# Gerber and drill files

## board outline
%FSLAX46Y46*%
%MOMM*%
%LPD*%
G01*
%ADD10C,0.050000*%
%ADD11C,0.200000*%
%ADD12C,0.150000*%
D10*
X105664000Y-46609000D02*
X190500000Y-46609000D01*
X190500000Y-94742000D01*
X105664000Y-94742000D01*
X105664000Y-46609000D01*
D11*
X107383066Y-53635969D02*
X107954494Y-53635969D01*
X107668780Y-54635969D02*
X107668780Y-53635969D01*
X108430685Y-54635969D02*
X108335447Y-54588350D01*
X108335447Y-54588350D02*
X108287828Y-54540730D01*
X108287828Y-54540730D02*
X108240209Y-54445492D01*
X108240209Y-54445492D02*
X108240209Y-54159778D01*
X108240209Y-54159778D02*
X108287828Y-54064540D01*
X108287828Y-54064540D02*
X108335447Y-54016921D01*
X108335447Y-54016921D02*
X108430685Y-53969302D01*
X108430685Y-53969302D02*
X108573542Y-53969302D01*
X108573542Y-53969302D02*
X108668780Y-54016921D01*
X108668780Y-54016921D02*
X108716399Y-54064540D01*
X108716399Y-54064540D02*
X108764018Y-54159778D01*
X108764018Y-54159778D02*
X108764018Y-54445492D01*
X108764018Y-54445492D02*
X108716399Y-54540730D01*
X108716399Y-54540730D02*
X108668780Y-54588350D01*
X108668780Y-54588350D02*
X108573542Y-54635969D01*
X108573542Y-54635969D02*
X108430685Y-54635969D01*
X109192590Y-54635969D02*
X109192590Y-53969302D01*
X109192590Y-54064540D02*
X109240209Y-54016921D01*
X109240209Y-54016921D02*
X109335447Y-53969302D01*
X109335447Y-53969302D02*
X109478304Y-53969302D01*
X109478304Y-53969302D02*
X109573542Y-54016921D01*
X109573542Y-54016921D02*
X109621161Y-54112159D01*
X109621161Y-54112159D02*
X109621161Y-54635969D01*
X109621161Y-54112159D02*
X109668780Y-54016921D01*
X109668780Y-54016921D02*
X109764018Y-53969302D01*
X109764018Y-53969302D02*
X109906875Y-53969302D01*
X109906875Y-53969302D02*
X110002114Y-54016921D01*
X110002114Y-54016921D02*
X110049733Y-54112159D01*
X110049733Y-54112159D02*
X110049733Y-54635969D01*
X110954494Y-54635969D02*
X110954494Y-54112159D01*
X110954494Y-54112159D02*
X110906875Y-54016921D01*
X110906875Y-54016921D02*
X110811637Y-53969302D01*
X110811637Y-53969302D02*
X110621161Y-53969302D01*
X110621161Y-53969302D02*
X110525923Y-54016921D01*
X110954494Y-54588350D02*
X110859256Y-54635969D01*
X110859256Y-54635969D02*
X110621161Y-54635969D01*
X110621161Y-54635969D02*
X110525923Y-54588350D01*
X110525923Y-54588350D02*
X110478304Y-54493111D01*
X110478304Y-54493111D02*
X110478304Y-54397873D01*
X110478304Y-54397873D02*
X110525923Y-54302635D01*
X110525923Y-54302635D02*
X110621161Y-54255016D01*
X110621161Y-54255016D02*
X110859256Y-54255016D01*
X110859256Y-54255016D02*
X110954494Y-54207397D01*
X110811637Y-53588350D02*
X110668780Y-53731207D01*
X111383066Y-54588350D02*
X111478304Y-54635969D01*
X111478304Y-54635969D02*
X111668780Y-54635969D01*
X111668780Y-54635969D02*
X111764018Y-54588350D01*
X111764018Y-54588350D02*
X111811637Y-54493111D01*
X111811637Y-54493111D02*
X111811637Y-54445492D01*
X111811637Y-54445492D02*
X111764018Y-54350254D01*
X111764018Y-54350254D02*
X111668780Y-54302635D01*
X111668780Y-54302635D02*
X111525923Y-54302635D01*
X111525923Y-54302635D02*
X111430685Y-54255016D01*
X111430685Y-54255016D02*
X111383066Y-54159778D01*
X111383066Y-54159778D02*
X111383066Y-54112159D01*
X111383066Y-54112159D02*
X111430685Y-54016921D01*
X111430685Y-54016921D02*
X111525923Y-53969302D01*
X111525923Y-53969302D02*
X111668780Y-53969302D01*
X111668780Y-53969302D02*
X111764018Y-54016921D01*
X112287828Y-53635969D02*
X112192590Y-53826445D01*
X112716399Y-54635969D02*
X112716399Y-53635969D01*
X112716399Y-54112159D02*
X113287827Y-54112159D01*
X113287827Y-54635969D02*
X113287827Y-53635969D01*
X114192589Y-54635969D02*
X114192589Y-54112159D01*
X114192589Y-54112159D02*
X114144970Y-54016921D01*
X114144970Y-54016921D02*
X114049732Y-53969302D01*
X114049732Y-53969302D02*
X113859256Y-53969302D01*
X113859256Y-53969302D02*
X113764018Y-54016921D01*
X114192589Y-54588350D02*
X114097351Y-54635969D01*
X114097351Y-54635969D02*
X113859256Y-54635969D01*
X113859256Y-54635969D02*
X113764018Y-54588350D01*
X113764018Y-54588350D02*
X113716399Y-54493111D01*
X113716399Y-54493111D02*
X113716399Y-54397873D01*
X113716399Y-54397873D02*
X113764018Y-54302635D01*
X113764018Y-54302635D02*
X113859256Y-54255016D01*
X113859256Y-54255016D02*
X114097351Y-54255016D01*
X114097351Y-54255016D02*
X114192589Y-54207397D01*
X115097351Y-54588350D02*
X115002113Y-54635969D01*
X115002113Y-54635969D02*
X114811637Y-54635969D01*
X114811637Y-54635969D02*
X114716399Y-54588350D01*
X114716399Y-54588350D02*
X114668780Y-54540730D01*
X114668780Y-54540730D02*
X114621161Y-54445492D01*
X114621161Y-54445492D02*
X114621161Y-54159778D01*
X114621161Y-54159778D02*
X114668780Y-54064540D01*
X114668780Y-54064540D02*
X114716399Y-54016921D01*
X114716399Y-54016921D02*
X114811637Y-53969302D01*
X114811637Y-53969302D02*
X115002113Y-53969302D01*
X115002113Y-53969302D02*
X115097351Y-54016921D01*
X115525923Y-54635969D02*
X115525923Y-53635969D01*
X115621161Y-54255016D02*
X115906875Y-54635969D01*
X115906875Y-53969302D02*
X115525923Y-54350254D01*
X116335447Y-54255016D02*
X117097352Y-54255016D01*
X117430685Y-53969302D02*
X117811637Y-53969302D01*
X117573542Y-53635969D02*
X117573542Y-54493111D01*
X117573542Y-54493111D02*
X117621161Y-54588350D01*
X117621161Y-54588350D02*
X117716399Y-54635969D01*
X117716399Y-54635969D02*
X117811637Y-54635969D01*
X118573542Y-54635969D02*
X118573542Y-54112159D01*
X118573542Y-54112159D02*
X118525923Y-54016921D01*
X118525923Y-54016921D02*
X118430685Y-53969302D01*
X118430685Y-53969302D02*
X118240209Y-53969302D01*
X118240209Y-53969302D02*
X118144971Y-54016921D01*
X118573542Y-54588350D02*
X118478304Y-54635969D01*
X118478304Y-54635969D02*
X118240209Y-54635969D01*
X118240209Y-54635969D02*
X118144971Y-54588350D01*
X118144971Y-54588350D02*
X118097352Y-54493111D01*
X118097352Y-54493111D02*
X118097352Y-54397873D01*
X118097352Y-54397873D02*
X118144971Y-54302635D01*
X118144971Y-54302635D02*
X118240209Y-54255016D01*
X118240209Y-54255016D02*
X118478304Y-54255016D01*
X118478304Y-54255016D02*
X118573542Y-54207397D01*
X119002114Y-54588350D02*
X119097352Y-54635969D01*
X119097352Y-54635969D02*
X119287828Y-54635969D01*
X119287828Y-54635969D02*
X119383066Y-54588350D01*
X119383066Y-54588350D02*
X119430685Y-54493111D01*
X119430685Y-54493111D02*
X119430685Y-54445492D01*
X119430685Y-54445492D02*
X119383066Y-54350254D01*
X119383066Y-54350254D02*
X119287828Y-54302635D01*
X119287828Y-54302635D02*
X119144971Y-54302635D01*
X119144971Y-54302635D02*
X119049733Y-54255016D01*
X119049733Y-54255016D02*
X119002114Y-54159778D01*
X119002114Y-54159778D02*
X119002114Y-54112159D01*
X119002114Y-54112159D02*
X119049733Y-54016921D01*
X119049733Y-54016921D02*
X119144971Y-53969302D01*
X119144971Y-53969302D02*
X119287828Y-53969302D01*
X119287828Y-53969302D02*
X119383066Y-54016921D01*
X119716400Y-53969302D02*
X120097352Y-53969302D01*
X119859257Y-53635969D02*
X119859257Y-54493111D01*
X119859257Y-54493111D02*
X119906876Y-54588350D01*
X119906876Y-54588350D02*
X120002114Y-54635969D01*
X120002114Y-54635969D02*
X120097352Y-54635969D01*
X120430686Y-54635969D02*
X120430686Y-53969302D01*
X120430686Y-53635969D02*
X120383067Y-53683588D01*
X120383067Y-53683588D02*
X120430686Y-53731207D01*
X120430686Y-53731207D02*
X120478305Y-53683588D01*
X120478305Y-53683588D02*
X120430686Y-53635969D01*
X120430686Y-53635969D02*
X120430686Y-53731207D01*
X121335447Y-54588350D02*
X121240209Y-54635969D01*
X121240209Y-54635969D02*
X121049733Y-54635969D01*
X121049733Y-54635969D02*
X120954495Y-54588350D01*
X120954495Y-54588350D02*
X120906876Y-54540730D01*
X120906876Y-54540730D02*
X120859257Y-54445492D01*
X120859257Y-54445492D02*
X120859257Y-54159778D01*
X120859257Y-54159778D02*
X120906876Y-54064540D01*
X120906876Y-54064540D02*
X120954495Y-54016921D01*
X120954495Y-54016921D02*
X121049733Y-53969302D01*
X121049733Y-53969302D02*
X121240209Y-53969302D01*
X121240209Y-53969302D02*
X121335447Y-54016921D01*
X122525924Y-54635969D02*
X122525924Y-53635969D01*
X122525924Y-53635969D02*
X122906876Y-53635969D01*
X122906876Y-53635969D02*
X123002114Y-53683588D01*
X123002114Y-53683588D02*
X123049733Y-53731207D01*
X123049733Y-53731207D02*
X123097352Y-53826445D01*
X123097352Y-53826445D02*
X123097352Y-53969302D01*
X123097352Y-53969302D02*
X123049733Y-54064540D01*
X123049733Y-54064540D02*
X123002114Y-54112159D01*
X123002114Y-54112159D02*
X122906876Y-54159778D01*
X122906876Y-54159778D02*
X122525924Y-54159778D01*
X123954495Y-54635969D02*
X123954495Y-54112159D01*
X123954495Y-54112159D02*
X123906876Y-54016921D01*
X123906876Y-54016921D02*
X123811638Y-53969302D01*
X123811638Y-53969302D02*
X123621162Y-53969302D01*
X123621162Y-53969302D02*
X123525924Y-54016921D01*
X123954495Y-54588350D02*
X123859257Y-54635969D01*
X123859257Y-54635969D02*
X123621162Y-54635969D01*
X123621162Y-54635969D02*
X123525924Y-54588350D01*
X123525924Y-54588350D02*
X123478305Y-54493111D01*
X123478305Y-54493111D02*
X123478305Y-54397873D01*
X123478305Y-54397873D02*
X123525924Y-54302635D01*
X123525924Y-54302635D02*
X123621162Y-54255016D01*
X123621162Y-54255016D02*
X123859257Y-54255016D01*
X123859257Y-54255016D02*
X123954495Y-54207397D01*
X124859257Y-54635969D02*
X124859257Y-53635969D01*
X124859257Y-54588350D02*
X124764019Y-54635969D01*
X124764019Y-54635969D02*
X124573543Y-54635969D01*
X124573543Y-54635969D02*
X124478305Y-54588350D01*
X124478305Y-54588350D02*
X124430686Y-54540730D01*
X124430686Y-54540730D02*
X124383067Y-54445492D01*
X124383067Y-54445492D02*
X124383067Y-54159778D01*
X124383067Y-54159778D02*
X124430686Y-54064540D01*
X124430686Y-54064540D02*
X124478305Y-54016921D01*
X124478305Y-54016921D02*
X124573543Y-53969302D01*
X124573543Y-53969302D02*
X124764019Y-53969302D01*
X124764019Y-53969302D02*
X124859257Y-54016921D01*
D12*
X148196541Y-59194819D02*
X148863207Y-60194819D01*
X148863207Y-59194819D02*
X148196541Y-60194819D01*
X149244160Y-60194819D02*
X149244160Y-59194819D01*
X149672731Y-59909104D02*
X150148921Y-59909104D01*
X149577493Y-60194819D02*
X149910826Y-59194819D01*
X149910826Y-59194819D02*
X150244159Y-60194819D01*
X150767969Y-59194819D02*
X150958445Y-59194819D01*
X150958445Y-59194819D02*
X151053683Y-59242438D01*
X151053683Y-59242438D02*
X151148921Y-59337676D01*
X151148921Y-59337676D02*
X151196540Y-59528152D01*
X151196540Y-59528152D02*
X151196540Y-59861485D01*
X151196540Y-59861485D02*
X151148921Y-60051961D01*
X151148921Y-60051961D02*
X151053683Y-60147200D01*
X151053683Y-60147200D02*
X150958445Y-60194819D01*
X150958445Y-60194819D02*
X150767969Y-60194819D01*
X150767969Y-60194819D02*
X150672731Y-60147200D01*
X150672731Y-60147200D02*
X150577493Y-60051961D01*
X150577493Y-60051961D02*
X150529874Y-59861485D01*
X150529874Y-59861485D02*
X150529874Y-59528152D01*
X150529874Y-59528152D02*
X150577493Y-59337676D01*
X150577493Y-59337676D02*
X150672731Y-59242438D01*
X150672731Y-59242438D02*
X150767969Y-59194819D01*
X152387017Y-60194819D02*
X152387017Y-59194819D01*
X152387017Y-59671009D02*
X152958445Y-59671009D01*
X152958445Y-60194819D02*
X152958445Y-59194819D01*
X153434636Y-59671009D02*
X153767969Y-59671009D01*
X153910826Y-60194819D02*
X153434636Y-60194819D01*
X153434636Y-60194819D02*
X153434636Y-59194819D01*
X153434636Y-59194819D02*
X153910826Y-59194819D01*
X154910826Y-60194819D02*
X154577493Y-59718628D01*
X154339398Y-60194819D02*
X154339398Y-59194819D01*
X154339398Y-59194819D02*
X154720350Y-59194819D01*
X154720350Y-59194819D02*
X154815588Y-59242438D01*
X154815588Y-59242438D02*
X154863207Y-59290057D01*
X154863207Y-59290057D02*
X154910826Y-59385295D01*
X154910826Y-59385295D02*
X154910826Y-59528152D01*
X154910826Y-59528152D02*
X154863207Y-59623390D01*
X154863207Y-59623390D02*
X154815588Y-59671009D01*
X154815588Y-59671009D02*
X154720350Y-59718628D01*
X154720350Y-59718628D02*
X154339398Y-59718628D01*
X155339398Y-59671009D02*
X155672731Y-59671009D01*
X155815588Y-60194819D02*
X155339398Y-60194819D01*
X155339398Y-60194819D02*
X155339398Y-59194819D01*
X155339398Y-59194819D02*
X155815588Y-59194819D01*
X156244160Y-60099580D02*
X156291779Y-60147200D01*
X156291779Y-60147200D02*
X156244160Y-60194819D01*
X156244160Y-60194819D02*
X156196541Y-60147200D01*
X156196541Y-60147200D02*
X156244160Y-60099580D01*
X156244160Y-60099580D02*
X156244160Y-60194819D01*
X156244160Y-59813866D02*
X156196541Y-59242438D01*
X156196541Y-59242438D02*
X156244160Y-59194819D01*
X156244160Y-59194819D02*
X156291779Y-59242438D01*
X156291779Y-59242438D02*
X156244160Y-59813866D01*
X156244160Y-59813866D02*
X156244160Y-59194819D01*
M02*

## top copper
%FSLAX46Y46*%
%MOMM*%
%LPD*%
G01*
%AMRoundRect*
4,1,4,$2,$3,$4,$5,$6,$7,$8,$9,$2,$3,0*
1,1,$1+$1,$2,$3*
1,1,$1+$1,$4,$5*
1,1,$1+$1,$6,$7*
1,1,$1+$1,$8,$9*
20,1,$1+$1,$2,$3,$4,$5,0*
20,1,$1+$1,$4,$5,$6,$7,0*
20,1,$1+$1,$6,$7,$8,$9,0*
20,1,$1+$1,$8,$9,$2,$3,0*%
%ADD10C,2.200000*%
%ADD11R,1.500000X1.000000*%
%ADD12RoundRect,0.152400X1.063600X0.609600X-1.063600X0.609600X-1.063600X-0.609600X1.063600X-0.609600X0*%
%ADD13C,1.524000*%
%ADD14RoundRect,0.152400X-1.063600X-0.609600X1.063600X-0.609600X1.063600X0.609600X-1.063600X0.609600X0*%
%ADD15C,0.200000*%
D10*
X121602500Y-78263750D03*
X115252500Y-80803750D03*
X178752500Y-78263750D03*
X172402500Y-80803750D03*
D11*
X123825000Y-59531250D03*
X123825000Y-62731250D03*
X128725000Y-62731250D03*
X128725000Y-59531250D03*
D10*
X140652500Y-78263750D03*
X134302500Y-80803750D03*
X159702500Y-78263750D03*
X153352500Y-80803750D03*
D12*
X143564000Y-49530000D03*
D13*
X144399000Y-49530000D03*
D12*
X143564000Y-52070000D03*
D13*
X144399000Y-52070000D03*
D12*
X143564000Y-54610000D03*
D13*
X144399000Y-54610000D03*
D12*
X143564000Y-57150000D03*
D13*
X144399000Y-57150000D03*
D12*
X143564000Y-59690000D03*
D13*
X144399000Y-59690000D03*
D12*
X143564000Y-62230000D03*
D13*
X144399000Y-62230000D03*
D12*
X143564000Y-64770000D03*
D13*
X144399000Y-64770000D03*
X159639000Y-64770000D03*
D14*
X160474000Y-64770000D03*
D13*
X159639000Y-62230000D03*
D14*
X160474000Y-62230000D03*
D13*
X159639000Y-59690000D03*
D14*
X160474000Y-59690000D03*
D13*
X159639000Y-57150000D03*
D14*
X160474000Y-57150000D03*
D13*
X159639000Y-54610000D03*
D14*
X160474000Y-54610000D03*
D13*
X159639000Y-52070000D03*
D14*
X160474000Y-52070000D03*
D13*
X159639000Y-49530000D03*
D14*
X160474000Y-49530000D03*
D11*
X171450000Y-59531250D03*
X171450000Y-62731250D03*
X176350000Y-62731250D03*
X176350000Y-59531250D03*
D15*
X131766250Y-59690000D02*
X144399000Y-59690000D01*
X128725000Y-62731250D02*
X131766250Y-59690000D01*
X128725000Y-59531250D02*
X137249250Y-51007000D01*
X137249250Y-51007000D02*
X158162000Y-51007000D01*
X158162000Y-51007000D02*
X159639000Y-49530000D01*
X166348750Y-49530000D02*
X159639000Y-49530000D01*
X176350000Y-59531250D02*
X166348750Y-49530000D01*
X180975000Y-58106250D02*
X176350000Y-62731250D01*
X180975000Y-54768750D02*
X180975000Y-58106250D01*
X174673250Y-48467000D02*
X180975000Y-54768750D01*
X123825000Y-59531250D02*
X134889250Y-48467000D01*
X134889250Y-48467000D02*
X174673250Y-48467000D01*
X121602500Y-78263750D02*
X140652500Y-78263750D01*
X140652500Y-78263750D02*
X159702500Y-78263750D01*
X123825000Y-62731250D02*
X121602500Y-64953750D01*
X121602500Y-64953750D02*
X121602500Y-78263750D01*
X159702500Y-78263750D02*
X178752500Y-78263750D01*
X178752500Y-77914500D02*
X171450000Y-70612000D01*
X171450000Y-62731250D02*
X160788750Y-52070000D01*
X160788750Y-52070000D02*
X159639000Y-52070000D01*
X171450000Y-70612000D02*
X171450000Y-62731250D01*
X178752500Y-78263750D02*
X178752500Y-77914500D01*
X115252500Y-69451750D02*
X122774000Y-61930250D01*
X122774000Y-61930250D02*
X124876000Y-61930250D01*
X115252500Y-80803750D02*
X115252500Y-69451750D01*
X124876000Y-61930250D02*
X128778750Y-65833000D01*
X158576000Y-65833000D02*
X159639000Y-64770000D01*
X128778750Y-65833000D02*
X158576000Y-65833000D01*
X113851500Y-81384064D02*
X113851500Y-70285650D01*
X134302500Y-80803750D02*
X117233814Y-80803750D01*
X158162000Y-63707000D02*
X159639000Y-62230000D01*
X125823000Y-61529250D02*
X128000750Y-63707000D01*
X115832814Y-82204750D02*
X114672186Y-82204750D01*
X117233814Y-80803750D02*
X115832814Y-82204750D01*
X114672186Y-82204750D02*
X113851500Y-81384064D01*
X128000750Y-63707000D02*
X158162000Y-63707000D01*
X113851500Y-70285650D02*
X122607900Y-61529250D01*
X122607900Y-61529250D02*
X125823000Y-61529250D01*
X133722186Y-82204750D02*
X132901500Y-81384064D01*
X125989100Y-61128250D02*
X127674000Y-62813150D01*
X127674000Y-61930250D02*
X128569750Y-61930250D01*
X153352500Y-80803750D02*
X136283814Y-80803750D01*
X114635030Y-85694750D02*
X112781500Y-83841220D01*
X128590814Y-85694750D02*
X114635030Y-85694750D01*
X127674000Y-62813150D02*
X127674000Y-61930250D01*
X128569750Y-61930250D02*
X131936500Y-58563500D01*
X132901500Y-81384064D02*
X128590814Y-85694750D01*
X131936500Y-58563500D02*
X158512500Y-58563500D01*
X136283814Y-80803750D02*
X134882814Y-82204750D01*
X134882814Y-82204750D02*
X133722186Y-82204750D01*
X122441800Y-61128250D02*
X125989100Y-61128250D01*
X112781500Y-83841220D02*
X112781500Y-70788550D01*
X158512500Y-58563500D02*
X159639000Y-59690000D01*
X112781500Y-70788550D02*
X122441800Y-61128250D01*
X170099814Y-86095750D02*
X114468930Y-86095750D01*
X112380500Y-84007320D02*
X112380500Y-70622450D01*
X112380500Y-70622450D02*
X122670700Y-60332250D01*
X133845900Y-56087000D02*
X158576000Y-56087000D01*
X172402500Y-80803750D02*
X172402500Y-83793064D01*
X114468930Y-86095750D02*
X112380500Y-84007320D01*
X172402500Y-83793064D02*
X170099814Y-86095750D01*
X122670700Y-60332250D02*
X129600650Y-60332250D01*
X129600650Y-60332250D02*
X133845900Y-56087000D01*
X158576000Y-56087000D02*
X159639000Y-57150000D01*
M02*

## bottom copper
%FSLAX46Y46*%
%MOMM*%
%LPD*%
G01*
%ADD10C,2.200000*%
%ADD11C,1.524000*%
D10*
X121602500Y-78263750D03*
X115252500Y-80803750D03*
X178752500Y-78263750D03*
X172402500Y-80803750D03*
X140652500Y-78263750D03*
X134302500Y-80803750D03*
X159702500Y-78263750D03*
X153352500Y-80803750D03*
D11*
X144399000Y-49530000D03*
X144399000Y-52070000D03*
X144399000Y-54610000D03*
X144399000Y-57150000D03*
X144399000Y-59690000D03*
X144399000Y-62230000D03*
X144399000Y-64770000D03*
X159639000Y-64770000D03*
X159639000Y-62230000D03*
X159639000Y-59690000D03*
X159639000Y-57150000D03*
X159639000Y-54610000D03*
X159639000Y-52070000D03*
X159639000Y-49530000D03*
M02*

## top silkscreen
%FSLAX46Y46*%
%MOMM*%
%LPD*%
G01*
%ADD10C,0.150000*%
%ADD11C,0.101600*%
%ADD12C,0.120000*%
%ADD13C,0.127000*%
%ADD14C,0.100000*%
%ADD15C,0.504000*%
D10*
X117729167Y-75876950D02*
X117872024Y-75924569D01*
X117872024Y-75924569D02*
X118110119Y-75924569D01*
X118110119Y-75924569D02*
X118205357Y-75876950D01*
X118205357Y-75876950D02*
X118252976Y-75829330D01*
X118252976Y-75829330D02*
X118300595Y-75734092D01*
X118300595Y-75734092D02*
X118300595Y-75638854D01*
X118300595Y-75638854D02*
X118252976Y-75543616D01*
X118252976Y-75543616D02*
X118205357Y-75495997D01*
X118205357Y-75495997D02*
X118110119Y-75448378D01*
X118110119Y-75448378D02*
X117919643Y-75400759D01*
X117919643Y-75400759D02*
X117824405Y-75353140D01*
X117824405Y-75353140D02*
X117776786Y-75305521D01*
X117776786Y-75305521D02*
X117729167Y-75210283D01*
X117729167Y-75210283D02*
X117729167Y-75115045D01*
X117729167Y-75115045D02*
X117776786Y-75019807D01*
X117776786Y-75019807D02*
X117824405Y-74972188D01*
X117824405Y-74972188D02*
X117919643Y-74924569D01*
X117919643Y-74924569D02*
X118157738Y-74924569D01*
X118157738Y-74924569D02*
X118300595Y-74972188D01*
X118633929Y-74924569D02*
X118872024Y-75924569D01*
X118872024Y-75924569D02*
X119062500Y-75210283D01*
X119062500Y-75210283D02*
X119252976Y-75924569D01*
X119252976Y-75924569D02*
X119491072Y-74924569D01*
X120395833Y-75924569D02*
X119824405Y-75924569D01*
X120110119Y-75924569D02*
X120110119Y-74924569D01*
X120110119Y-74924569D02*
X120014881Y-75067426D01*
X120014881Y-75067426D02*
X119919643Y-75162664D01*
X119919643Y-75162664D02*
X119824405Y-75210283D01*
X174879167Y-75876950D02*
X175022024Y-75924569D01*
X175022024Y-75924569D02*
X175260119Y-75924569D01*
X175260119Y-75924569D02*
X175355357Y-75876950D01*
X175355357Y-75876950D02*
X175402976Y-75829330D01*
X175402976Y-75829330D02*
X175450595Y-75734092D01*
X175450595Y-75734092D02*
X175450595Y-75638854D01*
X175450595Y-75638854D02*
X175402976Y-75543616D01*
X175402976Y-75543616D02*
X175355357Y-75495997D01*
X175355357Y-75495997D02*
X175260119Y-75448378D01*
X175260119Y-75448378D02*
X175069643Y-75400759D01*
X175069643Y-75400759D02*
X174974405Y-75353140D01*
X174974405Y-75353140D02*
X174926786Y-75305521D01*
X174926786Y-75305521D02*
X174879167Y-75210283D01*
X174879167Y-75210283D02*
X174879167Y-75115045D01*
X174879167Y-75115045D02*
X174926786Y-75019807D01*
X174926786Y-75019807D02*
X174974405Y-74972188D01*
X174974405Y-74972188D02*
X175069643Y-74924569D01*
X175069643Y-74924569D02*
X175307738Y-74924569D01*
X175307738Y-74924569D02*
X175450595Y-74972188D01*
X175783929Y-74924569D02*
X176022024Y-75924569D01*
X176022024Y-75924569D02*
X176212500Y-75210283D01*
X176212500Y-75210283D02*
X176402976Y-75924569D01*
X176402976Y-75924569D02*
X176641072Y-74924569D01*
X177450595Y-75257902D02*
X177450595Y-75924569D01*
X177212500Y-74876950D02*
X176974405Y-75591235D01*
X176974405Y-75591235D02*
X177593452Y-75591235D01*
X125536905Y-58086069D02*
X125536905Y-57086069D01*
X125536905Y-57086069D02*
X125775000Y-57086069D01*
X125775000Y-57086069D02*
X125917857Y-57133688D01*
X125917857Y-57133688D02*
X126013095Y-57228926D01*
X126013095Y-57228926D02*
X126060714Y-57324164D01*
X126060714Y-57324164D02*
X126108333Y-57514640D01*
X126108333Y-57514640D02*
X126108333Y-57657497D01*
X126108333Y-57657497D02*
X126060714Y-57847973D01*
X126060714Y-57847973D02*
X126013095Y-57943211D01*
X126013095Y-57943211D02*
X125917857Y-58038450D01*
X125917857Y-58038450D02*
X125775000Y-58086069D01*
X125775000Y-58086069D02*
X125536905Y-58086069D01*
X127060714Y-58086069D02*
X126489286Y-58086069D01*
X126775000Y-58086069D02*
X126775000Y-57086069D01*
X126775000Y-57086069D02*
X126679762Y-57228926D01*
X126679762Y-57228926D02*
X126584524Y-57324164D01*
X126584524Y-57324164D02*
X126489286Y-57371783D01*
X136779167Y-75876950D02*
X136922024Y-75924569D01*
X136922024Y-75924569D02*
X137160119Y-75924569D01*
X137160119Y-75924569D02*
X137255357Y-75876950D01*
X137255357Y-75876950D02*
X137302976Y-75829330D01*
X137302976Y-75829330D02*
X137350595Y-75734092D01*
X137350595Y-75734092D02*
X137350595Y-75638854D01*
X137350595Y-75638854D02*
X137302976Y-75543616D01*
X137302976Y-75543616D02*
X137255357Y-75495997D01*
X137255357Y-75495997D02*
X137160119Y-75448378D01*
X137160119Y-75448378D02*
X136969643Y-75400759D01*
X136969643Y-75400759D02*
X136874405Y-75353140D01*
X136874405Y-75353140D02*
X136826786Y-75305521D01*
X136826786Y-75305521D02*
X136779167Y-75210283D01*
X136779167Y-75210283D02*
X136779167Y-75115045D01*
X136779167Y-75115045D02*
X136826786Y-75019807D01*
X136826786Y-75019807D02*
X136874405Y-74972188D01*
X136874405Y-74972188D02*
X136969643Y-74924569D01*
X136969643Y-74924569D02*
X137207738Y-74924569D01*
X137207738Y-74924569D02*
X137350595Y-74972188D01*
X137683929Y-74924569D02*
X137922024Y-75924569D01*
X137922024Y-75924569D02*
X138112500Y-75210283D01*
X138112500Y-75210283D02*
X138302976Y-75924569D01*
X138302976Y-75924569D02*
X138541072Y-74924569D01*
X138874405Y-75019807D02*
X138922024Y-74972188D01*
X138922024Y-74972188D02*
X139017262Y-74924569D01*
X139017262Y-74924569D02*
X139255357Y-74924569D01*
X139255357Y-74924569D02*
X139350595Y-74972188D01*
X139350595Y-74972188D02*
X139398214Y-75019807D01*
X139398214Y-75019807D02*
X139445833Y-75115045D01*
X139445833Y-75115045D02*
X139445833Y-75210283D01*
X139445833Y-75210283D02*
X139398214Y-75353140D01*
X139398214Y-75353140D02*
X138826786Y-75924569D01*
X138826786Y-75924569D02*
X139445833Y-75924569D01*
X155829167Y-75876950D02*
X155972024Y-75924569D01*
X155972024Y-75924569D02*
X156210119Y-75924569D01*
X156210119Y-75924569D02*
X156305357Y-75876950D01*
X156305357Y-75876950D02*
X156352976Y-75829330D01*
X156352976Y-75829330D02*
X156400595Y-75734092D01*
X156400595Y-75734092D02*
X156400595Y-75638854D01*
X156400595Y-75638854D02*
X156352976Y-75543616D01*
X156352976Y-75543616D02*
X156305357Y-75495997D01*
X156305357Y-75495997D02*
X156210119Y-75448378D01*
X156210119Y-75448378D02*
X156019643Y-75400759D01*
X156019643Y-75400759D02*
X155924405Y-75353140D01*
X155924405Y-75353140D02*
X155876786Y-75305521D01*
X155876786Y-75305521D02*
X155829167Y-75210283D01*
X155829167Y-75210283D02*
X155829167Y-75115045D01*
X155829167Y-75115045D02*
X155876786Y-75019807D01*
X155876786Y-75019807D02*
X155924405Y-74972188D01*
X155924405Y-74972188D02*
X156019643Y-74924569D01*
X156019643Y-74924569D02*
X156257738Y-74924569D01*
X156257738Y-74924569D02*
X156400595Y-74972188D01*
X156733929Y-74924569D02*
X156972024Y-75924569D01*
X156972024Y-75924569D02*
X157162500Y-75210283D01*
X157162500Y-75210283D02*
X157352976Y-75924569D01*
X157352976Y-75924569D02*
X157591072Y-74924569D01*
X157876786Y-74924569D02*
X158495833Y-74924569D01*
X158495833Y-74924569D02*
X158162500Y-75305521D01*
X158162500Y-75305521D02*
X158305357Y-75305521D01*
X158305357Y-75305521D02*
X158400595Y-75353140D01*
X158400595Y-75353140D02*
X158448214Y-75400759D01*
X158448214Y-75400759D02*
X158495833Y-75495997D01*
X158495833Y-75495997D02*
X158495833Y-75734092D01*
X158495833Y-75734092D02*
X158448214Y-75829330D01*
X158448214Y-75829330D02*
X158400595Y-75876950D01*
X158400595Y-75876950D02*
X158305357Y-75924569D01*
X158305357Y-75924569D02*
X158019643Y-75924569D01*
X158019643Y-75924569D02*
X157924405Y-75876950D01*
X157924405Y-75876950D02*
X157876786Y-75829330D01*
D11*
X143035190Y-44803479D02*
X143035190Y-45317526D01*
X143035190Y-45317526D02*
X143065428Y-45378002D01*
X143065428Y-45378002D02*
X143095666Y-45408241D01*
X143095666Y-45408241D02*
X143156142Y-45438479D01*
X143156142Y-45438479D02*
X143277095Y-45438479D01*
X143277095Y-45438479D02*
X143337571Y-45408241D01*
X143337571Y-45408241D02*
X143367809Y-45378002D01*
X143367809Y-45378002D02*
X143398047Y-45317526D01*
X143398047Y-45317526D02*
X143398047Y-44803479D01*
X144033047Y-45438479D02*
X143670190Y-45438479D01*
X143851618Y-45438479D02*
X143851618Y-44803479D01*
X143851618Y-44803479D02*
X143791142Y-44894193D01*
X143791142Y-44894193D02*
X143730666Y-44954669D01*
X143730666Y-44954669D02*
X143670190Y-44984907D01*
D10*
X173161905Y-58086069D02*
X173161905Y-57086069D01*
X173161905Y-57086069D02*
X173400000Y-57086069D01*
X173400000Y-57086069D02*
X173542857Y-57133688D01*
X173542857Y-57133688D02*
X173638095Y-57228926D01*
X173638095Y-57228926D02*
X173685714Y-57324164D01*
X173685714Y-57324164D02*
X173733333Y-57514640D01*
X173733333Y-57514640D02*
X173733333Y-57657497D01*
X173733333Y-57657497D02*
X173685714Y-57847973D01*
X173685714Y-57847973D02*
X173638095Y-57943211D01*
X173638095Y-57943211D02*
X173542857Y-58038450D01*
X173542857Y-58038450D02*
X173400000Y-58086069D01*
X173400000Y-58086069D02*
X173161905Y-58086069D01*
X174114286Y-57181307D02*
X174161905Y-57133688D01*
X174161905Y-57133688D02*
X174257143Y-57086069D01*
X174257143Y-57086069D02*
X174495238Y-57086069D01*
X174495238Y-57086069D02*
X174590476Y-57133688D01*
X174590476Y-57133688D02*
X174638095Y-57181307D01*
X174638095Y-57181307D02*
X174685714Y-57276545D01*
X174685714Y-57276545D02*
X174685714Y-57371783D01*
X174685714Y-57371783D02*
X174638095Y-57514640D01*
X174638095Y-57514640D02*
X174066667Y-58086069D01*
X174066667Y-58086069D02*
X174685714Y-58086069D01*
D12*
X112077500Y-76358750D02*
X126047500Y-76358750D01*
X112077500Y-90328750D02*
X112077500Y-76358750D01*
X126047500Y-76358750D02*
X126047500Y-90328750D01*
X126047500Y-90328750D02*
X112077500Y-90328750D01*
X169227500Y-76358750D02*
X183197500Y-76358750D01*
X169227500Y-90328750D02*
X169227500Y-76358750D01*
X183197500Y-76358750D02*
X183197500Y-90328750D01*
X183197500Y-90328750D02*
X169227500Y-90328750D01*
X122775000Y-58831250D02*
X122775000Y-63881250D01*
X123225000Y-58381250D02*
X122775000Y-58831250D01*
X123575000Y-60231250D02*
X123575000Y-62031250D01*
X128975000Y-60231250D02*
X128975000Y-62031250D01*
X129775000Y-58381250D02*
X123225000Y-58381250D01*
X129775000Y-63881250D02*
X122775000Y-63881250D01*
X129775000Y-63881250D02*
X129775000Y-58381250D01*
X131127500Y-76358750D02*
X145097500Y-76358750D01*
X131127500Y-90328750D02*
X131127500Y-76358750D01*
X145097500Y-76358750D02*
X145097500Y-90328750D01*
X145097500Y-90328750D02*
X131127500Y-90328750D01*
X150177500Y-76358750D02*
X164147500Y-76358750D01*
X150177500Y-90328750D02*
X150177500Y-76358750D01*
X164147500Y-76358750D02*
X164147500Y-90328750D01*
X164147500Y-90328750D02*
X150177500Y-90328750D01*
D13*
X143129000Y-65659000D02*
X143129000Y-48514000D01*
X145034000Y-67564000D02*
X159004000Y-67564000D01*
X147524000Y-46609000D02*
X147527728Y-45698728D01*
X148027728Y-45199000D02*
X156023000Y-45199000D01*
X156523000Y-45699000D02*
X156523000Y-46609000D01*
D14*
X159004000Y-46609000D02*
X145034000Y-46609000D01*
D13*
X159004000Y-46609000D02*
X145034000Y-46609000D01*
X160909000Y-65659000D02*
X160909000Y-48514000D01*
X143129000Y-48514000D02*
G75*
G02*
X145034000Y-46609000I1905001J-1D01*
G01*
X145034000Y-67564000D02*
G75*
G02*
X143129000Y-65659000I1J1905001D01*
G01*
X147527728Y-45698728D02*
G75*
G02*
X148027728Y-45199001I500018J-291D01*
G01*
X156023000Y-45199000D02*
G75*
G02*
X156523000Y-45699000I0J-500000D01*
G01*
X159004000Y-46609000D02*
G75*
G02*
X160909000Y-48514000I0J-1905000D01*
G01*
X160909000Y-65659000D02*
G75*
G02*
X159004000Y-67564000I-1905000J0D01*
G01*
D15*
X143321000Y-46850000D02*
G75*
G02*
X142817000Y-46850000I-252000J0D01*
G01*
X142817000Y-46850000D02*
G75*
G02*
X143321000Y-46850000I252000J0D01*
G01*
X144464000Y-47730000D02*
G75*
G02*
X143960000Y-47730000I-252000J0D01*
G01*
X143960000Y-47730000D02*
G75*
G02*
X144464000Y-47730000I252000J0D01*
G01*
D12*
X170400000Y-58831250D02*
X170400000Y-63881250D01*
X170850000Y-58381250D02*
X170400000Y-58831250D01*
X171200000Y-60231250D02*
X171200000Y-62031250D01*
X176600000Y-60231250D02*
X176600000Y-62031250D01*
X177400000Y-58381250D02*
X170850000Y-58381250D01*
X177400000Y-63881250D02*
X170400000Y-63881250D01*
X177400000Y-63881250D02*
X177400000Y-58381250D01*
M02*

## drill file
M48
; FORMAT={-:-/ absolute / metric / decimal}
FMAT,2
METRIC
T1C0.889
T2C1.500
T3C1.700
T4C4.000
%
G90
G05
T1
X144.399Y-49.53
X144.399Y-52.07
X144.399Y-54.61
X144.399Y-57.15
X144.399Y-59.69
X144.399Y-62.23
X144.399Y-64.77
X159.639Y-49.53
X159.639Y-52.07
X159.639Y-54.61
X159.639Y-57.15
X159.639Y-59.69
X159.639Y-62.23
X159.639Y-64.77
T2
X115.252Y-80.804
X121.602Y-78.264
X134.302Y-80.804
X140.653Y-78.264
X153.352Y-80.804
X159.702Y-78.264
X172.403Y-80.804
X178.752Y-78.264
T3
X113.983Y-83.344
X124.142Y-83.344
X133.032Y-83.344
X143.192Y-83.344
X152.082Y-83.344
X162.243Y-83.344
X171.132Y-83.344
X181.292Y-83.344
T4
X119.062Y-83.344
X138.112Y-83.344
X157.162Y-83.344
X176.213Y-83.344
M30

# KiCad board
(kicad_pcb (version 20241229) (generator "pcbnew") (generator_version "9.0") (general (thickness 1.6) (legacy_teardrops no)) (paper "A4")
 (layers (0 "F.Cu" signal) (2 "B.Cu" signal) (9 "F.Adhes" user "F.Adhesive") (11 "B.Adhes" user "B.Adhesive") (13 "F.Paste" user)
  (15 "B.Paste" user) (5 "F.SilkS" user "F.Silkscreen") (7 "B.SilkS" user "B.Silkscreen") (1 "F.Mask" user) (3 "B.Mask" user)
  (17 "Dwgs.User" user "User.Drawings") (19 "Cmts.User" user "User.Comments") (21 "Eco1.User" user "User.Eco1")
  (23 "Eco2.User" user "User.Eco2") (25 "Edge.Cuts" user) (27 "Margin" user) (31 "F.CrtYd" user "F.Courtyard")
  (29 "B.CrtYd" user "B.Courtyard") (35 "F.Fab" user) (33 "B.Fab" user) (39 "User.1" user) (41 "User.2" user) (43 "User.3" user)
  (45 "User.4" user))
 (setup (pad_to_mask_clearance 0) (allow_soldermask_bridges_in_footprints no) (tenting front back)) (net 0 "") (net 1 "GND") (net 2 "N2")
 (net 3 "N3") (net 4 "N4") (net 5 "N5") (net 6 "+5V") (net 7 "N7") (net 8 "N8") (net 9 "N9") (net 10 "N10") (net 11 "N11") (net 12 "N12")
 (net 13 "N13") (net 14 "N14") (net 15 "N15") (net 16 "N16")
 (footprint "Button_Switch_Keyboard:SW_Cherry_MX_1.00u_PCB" (layer "F.Cu") (at 121.6025 78.26375)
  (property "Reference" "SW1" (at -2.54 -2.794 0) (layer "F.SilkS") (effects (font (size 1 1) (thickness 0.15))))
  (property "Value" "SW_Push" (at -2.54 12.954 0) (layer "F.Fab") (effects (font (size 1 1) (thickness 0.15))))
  (fp_line (start -9.525 -1.905) (end 4.445 -1.905) (stroke (width 0.12) (type solid)) (layer "F.SilkS"))
  (fp_line (start -9.525 12.065) (end -9.525 -1.905) (stroke (width 0.12) (type solid)) (layer "F.SilkS"))
  (fp_line (start 4.445 -1.905) (end 4.445 12.065) (stroke (width 0.12) (type solid)) (layer "F.SilkS"))
  (fp_line (start 4.445 12.065) (end -9.525 12.065) (stroke (width 0.12) (type solid)) (layer "F.SilkS"))
  (pad "" np_thru_hole circle (at -7.62 5.08) (size 1.7 1.7) (drill 1.7) (layers "*.Cu" "*.Mask"))
  (pad "" np_thru_hole circle (at -2.54 5.08) (size 4 4) (drill 4) (layers "*.Cu" "*.Mask"))
  (pad "" np_thru_hole circle (at 2.54 5.08) (size 1.7 1.7) (drill 1.7) (layers "*.Cu" "*.Mask"))
  (pad "1" thru_hole circle (at 0 0) (size 2.2 2.2) (drill 1.5) (layers "*.Cu" "*.Mask") (remove_unused_layers no) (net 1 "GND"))
  (pad "2" thru_hole circle (at -6.35 2.54) (size 2.2 2.2) (drill 1.5) (layers "*.Cu" "*.Mask") (remove_unused_layers no) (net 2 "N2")))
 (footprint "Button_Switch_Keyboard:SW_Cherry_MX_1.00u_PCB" (layer "F.Cu") (at 178.7525 78.26375)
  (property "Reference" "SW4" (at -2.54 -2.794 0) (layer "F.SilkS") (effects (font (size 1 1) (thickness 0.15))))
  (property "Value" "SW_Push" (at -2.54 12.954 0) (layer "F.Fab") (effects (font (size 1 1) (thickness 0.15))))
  (fp_line (start -9.525 -1.905) (end 4.445 -1.905) (stroke (width 0.12) (type solid)) (layer "F.SilkS"))
  (fp_line (start -9.525 12.065) (end -9.525 -1.905) (stroke (width 0.12) (type solid)) (layer "F.SilkS"))
  (fp_line (start 4.445 -1.905) (end 4.445 12.065) (stroke (width 0.12) (type solid)) (layer "F.SilkS"))
  (fp_line (start 4.445 12.065) (end -9.525 12.065) (stroke (width 0.12) (type solid)) (layer "F.SilkS"))
  (pad "" np_thru_hole circle (at -7.62 5.08) (size 1.7 1.7) (drill 1.7) (layers "*.Cu" "*.Mask"))
  (pad "" np_thru_hole circle (at -2.54 5.08) (size 4 4) (drill 4) (layers "*.Cu" "*.Mask"))
  (pad "" np_thru_hole circle (at 2.54 5.08) (size 1.7 1.7) (drill 1.7) (layers "*.Cu" "*.Mask"))
  (pad "1" thru_hole circle (at 0 0) (size 2.2 2.2) (drill 1.5) (layers "*.Cu" "*.Mask") (remove_unused_layers no) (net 1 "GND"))
  (pad "2" thru_hole circle (at -6.35 2.54) (size 2.2 2.2) (drill 1.5) (layers "*.Cu" "*.Mask") (remove_unused_layers no) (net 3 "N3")))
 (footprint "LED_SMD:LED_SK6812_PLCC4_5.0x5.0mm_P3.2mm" (layer "F.Cu") (at 126.275 61.13125)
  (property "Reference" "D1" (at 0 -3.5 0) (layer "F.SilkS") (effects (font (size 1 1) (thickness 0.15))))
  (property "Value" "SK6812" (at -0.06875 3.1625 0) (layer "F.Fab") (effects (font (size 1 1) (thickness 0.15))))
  (fp_line (start -3.5 -2.3) (end -3.5 2.75) (stroke (width 0.12) (type default)) (layer "F.SilkS"))
  (fp_line (start -3.05 -2.75) (end -3.5 -2.3) (stroke (width 0.12) (type default)) (layer "F.SilkS"))
  (fp_line (start -2.7 -0.9) (end -2.7 0.9) (stroke (width 0.12) (type default)) (layer "F.SilkS"))
  (fp_line (start 2.7 -0.9) (end 2.7 0.9) (stroke (width 0.12) (type default)) (layer "F.SilkS"))
  (fp_line (start 3.5 -2.75) (end -3.05 -2.75) (stroke (width 0.12) (type solid)) (layer "F.SilkS"))
  (fp_line (start 3.5 2.75) (end -3.5 2.75) (stroke (width 0.12) (type solid)) (layer "F.SilkS"))
  (fp_line (start 3.5 2.75) (end 3.5 -2.75) (stroke (width 0.12) (type default)) (layer "F.SilkS"))
  (pad "1" smd rect (at -2.45 -1.6 180) (size 1.5 1) (layers "F.Cu" "F.Mask" "F.Paste") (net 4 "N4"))
  (pad "2" smd rect (at -2.45 1.6 180) (size 1.5 1) (layers "F.Cu" "F.Mask" "F.Paste") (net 1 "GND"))
  (pad "3" smd rect (at 2.45 1.6 180) (size 1.5 1) (layers "F.Cu" "F.Mask" "F.Paste") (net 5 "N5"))
  (pad "4" smd rect (at 2.45 -1.6 180) (size 1.5 1) (layers "F.Cu" "F.Mask" "F.Paste") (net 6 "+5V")))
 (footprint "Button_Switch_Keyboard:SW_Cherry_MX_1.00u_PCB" (layer "F.Cu") (at 140.6525 78.26375)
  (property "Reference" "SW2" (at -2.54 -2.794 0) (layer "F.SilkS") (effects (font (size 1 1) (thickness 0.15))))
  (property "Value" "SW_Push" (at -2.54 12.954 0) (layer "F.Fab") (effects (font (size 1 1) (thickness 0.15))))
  (fp_line (start -9.525 -1.905) (end 4.445 -1.905) (stroke (width 0.12) (type solid)) (layer "F.SilkS"))
  (fp_line (start -9.525 12.065) (end -9.525 -1.905) (stroke (width 0.12) (type solid)) (layer "F.SilkS"))
  (fp_line (start 4.445 -1.905) (end 4.445 12.065) (stroke (width 0.12) (type solid)) (layer "F.SilkS"))
  (fp_line (start 4.445 12.065) (end -9.525 12.065) (stroke (width 0.12) (type solid)) (layer "F.SilkS"))
  (pad "" np_thru_hole circle (at -7.62 5.08) (size 1.7 1.7) (drill 1.7) (layers "*.Cu" "*.Mask"))
  (pad "" np_thru_hole circle (at -2.54 5.08) (size 4 4) (drill 4) (layers "*.Cu" "*.Mask"))
  (pad "" np_thru_hole circle (at 2.54 5.08) (size 1.7 1.7) (drill 1.7) (layers "*.Cu" "*.Mask"))
  (pad "1" thru_hole circle (at 0 0) (size 2.2 2.2) (drill 1.5) (layers "*.Cu" "*.Mask") (remove_unused_layers no) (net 1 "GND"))
  (pad "2" thru_hole circle (at -6.35 2.54) (size 2.2 2.2) (drill 1.5) (layers "*.Cu" "*.Mask") (remove_unused_layers no) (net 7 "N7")))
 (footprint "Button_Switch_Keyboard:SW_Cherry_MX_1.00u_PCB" (layer "F.Cu") (at 159.7025 78.26375)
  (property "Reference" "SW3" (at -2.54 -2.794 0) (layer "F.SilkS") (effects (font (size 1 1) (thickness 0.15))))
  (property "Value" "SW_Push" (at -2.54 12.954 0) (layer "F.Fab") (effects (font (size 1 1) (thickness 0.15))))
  (fp_line (start -9.525 -1.905) (end 4.445 -1.905) (stroke (width 0.12) (type solid)) (layer "F.SilkS"))
  (fp_line (start -9.525 12.065) (end -9.525 -1.905) (stroke (width 0.12) (type solid)) (layer "F.SilkS"))
  (fp_line (start 4.445 -1.905) (end 4.445 12.065) (stroke (width 0.12) (type solid)) (layer "F.SilkS"))
  (fp_line (start 4.445 12.065) (end -9.525 12.065) (stroke (width 0.12) (type solid)) (layer "F.SilkS"))
  (pad "" np_thru_hole circle (at -7.62 5.08) (size 1.7 1.7) (drill 1.7) (layers "*.Cu" "*.Mask"))
  (pad "" np_thru_hole circle (at -2.54 5.08) (size 4 4) (drill 4) (layers "*.Cu" "*.Mask"))
  (pad "" np_thru_hole circle (at 2.54 5.08) (size 1.7 1.7) (drill 1.7) (layers "*.Cu" "*.Mask"))
  (pad "1" thru_hole circle (at 0 0) (size 2.2 2.2) (drill 1.5) (layers "*.Cu" "*.Mask") (remove_unused_layers no) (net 1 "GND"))
  (pad "2" thru_hole circle (at -6.35 2.54) (size 2.2 2.2) (drill 1.5) (layers "*.Cu" "*.Mask") (remove_unused_layers no) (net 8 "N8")))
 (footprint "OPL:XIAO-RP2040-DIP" (layer "F.Cu") (at 152.019 57.15)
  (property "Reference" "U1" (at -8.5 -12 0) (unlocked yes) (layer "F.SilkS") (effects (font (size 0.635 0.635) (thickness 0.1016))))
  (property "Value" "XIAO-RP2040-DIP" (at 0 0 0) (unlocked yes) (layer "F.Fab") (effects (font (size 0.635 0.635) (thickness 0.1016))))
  (fp_line (start -8.89 8.509) (end -8.89 -8.636) (stroke (width 0.127) (type solid)) (layer "F.SilkS"))
  (fp_line (start -6.985 10.414) (end 6.985 10.414) (stroke (width 0.127) (type solid)) (layer "F.SilkS"))
  (fp_line (start -4.495 -10.541) (end -4.491272 -11.451272) (stroke (width 0.127) (type solid)) (layer "F.SilkS"))
  (fp_line (start -3.991272 -11.951) (end 4.004 -11.951) (stroke (width 0.127) (type solid)) (layer "F.SilkS"))
  (fp_line (start 4.504 -11.451) (end 4.504 -10.541) (stroke (width 0.127) (type solid)) (layer "F.SilkS"))
  (fp_line (start 6.985 -10.541) (end -6.985 -10.541) (stroke (width 0.1) (type solid)) (layer "F.SilkS"))
  (fp_line (start 6.985 -10.541) (end -6.985 -10.541) (stroke (width 0.127) (type solid)) (layer "F.SilkS"))
  (fp_line (start 8.89 8.509) (end 8.89 -8.636) (stroke (width 0.127) (type solid)) (layer "F.SilkS"))
  (fp_arc (start -8.89 -8.636) (mid -8.332038 -9.983038) (end -6.985 -10.541) (stroke (width 0.127) (type solid)) (layer "F.SilkS"))
  (fp_arc (start -6.985 10.414) (mid -8.332038 9.856038) (end -8.89 8.509) (stroke (width 0.127) (type solid)) (layer "F.SilkS"))
  (fp_arc (start -4.491272 -11.451272) (mid -4.344728 -11.80464) (end -3.991272 -11.951) (stroke (width 0.127) (type default))
   (layer "F.SilkS"))
  (fp_arc (start 4.004 -11.951) (mid 4.357553 -11.804553) (end 4.504 -11.451) (stroke (width 0.127) (type default)) (layer "F.SilkS"))
  (fp_arc (start 6.985 -10.541) (mid 8.332038 -9.983038) (end 8.89 -8.636) (stroke (width 0.127) (type solid)) (layer "F.SilkS"))
  (fp_arc (start 8.89 8.509) (mid 8.332038 9.856038) (end 6.985 10.414) (stroke (width 0.127) (type solid)) (layer "F.SilkS"))
  (fp_circle (center -8.95 -10.3) (end -8.95 -10.554) (stroke (width 0.5) (type solid)) (fill yes) (layer "F.SilkS"))
  (fp_circle (center -7.807 -9.42) (end -7.807 -9.674) (stroke (width 0.5) (type solid)) (fill yes) (layer "F.SilkS"))
  (pad "1" smd roundrect (at -8.455 -7.62 180) (size 2.432 1.524) (layers "F.Cu" "F.Mask") (roundrect_rratio 0.1) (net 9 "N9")
   (thermal_bridge_angle 45))
  (pad "1" thru_hole circle (at -7.62 -7.62 180) (size 1.524 1.524) (drill 0.889) (layers "*.Cu" "*.Mask") (remove_unused_layers no)
   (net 9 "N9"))
  (pad "2" smd roundrect (at -8.455 -5.08 180) (size 2.432 1.524) (layers "F.Cu" "F.Mask") (roundrect_rratio 0.1) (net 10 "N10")
   (thermal_bridge_angle 45))
  (pad "2" thru_hole circle (at -7.62 -5.08 180) (size 1.524 1.524) (drill 0.889) (layers "*.Cu" "*.Mask") (remove_unused_layers no)
   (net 10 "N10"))
  (pad "3" smd roundrect (at -8.455 -2.54 180) (size 2.432 1.524) (layers "F.Cu" "F.Mask") (roundrect_rratio 0.1) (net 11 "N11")
   (thermal_bridge_angle 45))
  (pad "3" thru_hole circle (at -7.62 -2.54 180) (size 1.524 1.524) (drill 0.889) (layers "*.Cu" "*.Mask") (remove_unused_layers no)
   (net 11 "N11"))
  (pad "4" smd roundrect (at -8.455 0 180) (size 2.432 1.524) (layers "F.Cu" "F.Mask") (roundrect_rratio 0.1) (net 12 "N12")
   (thermal_bridge_angle 45))
  (pad "4" thru_hole circle (at -7.62 0 180) (size 1.524 1.524) (drill 0.889) (layers "*.Cu" "*.Mask") (remove_unused_layers no)
   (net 12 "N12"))
  (pad "5" smd roundrect (at -8.455 2.54 180) (size 2.432 1.524) (layers "F.Cu" "F.Mask") (roundrect_rratio 0.1) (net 5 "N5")
   (thermal_bridge_angle 45))
  (pad "5" thru_hole circle (at -7.62 2.54 180) (size 1.524 1.524) (drill 0.889) (layers "*.Cu" "*.Mask") (remove_unused_layers no)
   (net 5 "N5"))
  (pad "6" smd roundrect (at -8.455 5.08 180) (size 2.432 1.524) (layers "F.Cu" "F.Mask") (roundrect_rratio 0.1) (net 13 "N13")
   (thermal_bridge_angle 45))
  (pad "6" thru_hole circle (at -7.62 5.08 180) (size 1.524 1.524) (drill 0.889) (layers "*.Cu" "*.Mask") (remove_unused_layers no)
   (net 13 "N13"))
  (pad "7" smd roundrect (at -8.455 7.62 180) (size 2.432 1.524) (layers "F.Cu" "F.Mask") (roundrect_rratio 0.1) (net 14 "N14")
   (thermal_bridge_angle 45))
  (pad "7" thru_hole circle (at -7.62 7.62 180) (size 1.524 1.524) (drill 0.889) (layers "*.Cu" "*.Mask") (remove_unused_layers no)
   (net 14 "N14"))
  (pad "8" thru_hole circle (at 7.62 7.62) (size 1.524 1.524) (drill 0.889) (layers "*.Cu" "*.Mask") (remove_unused_layers no) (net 2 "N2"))
  (pad "8" smd roundrect (at 8.455 7.62) (size 2.432 1.524) (layers "F.Cu" "F.Mask") (roundrect_rratio 0.1) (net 2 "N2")
   (thermal_bridge_angle 45))
  (pad "9" thru_hole circle (at 7.62 5.08) (size 1.524 1.524) (drill 0.889) (layers "*.Cu" "*.Mask") (remove_unused_layers no) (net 7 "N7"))
  (pad "9" smd roundrect (at 8.455 5.08) (size 2.432 1.524) (layers "F.Cu" "F.Mask") (roundrect_rratio 0.1) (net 7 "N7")
   (thermal_bridge_angle 45))
  (pad "10" thru_hole circle (at 7.62 2.54) (size 1.524 1.524) (drill 0.889) (layers "*.Cu" "*.Mask") (remove_unused_layers no) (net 8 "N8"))
  (pad "10" smd roundrect (at 8.455 2.54) (size 2.432 1.524) (layers "F.Cu" "F.Mask") (roundrect_rratio 0.1) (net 8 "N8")
   (thermal_bridge_angle 45))
  (pad "11" thru_hole circle (at 7.62 0) (size 1.524 1.524) (drill 0.889) (layers "*.Cu" "*.Mask") (remove_unused_layers no) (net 3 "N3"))
  (pad "11" smd roundrect (at 8.455 0) (size 2.432 1.524) (layers "F.Cu" "F.Mask") (roundrect_rratio 0.1) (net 3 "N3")
   (thermal_bridge_angle 45))
  (pad "12" thru_hole circle (at 7.62 -2.54) (size 1.524 1.524) (drill 0.889) (layers "*.Cu" "*.Mask") (remove_unused_layers no)
   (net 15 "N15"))
  (pad "12" smd roundrect (at 8.455 -2.54) (size 2.432 1.524) (layers "F.Cu" "F.Mask") (roundrect_rratio 0.1) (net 15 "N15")
   (thermal_bridge_angle 45))
  (pad "13" thru_hole circle (at 7.62 -5.08) (size 1.524 1.524) (drill 0.889) (layers "*.Cu" "*.Mask") (remove_unused_layers no)
   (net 1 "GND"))
  (pad "13" smd roundrect (at 8.455 -5.08) (size 2.432 1.524) (layers "F.Cu" "F.Mask") (roundrect_rratio 0.1) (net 1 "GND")
   (thermal_bridge_angle 45))
  (pad "14" thru_hole circle (at 7.62 -7.62) (size 1.524 1.524) (drill 0.889) (layers "*.Cu" "*.Mask") (remove_unused_layers no)
   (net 6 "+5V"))
  (pad "14" smd roundrect (at 8.455 -7.62) (size 2.432 1.524) (layers "F.Cu" "F.Mask") (roundrect_rratio 0.1) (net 6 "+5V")
   (thermal_bridge_angle 45)))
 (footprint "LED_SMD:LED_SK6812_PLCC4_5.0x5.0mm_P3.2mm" (layer "F.Cu") (at 173.9 61.13125)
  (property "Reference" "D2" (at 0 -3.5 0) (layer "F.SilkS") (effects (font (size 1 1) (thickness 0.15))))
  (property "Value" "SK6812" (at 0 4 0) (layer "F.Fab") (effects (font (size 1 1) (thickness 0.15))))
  (fp_line (start -3.5 -2.3) (end -3.5 2.75) (stroke (width 0.12) (type default)) (layer "F.SilkS"))
  (fp_line (start -3.05 -2.75) (end -3.5 -2.3) (stroke (width 0.12) (type default)) (layer "F.SilkS"))
  (fp_line (start -2.7 -0.9) (end -2.7 0.9) (stroke (width 0.12) (type default)) (layer "F.SilkS"))
  (fp_line (start 2.7 -0.9) (end 2.7 0.9) (stroke (width 0.12) (type default)) (layer "F.SilkS"))
  (fp_line (start 3.5 -2.75) (end -3.05 -2.75) (stroke (width 0.12) (type solid)) (layer "F.SilkS"))
  (fp_line (start 3.5 2.75) (end -3.5 2.75) (stroke (width 0.12) (type solid)) (layer "F.SilkS"))
  (fp_line (start 3.5 2.75) (end 3.5 -2.75) (stroke (width 0.12) (type default)) (layer "F.SilkS"))
  (pad "1" smd rect (at -2.45 -1.6 180) (size 1.5 1) (layers "F.Cu" "F.Mask" "F.Paste") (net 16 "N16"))
  (pad "2" smd rect (at -2.45 1.6 180) (size 1.5 1) (layers "F.Cu" "F.Mask" "F.Paste") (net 1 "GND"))
  (pad "3" smd rect (at 2.45 1.6 180) (size 1.5 1) (layers "F.Cu" "F.Mask" "F.Paste") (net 4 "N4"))
  (pad "4" smd rect (at 2.45 -1.6 180) (size 1.5 1) (layers "F.Cu" "F.Mask" "F.Paste") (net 6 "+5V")))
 (gr_rect (start 105.664 46.609) (end 190.5 94.742) (stroke (width 0.05) (type default)) (fill no) (layer "Edge.Cuts"))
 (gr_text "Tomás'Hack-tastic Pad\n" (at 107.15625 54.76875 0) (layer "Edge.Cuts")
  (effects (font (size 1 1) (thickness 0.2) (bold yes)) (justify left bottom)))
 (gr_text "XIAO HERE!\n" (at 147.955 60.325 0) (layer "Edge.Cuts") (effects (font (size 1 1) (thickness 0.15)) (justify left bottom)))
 (segment (start 131.76625 59.69) (end 144.399 59.69) (width 0.2) (layer "F.Cu") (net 5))
 (segment (start 128.725 62.73125) (end 131.76625 59.69) (width 0.2) (layer "F.Cu") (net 5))
 (segment (start 128.725 59.53125) (end 137.24925 51.007) (width 0.2) (layer "F.Cu") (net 6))
 (segment (start 137.24925 51.007) (end 158.162 51.007) (width 0.2) (layer "F.Cu") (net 6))
 (segment (start 158.162 51.007) (end 159.639 49.53) (width 0.2) (layer "F.Cu") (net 6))
 (segment (start 166.34875 49.53) (end 159.639 49.53) (width 0.2) (layer "F.Cu") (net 6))
 (segment (start 176.35 59.53125) (end 166.34875 49.53) (width 0.2) (layer "F.Cu") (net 6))
 (segment (start 180.975 58.10625) (end 176.35 62.73125) (width 0.2) (layer "F.Cu") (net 4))
 (segment (start 180.975 54.76875) (end 180.975 58.10625) (width 0.2) (layer "F.Cu") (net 4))
 (segment (start 174.67325 48.467) (end 180.975 54.76875) (width 0.2) (layer "F.Cu") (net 4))
 (segment (start 123.825 59.53125) (end 134.88925 48.467) (width 0.2) (layer "F.Cu") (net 4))
 (segment (start 134.88925 48.467) (end 174.67325 48.467) (width 0.2) (layer "F.Cu") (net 4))
 (segment (start 121.6025 78.26375) (end 140.6525 78.26375) (width 0.2) (layer "F.Cu") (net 1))
 (segment (start 140.6525 78.26375) (end 159.7025 78.26375) (width 0.2) (layer "F.Cu") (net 1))
 (segment (start 123.825 62.73125) (end 121.6025 64.95375) (width 0.2) (layer "F.Cu") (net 1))
 (segment (start 121.6025 64.95375) (end 121.6025 78.26375) (width 0.2) (layer "F.Cu") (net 1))
 (segment (start 159.7025 78.26375) (end 178.7525 78.26375) (width 0.2) (layer "F.Cu") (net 1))
 (segment (start 178.7525 77.9145) (end 171.45 70.612) (width 0.2) (layer "F.Cu") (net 1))
 (segment (start 171.45 62.73125) (end 160.78875 52.07) (width 0.2) (layer "F.Cu") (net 1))
 (segment (start 160.78875 52.07) (end 159.639 52.07) (width 0.2) (layer "F.Cu") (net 1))
 (segment (start 171.45 70.612) (end 171.45 62.73125) (width 0.2) (layer "F.Cu") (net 1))
 (segment (start 178.7525 78.26375) (end 178.7525 77.9145) (width 0.2) (layer "F.Cu") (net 1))
 (segment (start 115.2525 69.45175) (end 122.774 61.93025) (width 0.2) (layer "F.Cu") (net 2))
 (segment (start 122.774 61.93025) (end 124.876 61.93025) (width 0.2) (layer "F.Cu") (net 2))
 (segment (start 115.2525 80.80375) (end 115.2525 69.45175) (width 0.2) (layer "F.Cu") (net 2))
 (segment (start 124.876 61.93025) (end 128.77875 65.833) (width 0.2) (layer "F.Cu") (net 2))
 (segment (start 158.576 65.833) (end 159.639 64.77) (width 0.2) (layer "F.Cu") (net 2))
 (segment (start 128.77875 65.833) (end 158.576 65.833) (width 0.2) (layer "F.Cu") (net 2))
 (segment (start 113.8515 81.384064) (end 113.8515 70.28565) (width 0.2) (layer "F.Cu") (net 7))
 (segment (start 134.3025 80.80375) (end 117.233814 80.80375) (width 0.2) (layer "F.Cu") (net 7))
 (segment (start 158.162 63.707) (end 159.639 62.23) (width 0.2) (layer "F.Cu") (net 7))
 (segment (start 125.823 61.52925) (end 128.00075 63.707) (width 0.2) (layer "F.Cu") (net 7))
 (segment (start 115.832814 82.20475) (end 114.672186 82.20475) (width 0.2) (layer "F.Cu") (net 7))
 (segment (start 117.233814 80.80375) (end 115.832814 82.20475) (width 0.2) (layer "F.Cu") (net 7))
 (segment (start 114.672186 82.20475) (end 113.8515 81.384064) (width 0.2) (layer "F.Cu") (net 7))
 (segment (start 128.00075 63.707) (end 158.162 63.707) (width 0.2) (layer "F.Cu") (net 7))
 (segment (start 113.8515 70.28565) (end 122.6079 61.52925) (width 0.2) (layer "F.Cu") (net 7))
 (segment (start 122.6079 61.52925) (end 125.823 61.52925) (width 0.2) (layer "F.Cu") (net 7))
 (segment (start 133.722186 82.20475) (end 132.9015 81.384064) (width 0.2) (layer "F.Cu") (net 8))
 (segment (start 125.9891 61.12825) (end 127.674 62.81315) (width 0.2) (layer "F.Cu") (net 8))
 (segment (start 127.674 61.93025) (end 128.56975 61.93025) (width 0.2) (layer "F.Cu") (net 8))
 (segment (start 153.3525 80.80375) (end 136.283814 80.80375) (width 0.2) (layer "F.Cu") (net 8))
 (segment (start 114.63503 85.69475) (end 112.7815 83.84122) (width 0.2) (layer "F.Cu") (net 8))
 (segment (start 128.590814 85.69475) (end 114.63503 85.69475) (width 0.2) (layer "F.Cu") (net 8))
 (segment (start 127.674 62.81315) (end 127.674 61.93025) (width 0.2) (layer "F.Cu") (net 8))
 (segment (start 128.56975 61.93025) (end 131.9365 58.5635) (width 0.2) (layer "F.Cu") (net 8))
 (segment (start 132.9015 81.384064) (end 128.590814 85.69475) (width 0.2) (layer "F.Cu") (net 8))
 (segment (start 131.9365 58.5635) (end 158.5125 58.5635) (width 0.2) (layer "F.Cu") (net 8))
 (segment (start 136.283814 80.80375) (end 134.882814 82.20475) (width 0.2) (layer "F.Cu") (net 8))
 (segment (start 134.882814 82.20475) (end 133.722186 82.20475) (width 0.2) (layer "F.Cu") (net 8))
 (segment (start 122.4418 61.12825) (end 125.9891 61.12825) (width 0.2) (layer "F.Cu") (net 8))
 (segment (start 112.7815 83.84122) (end 112.7815 70.78855) (width 0.2) (layer "F.Cu") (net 8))
 (segment (start 158.5125 58.5635) (end 159.639 59.69) (width 0.2) (layer "F.Cu") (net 8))
 (segment (start 112.7815 70.78855) (end 122.4418 61.12825) (width 0.2) (layer "F.Cu") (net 8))
 (segment (start 170.099814 86.09575) (end 114.46893 86.09575) (width 0.2) (layer "F.Cu") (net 3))
 (segment (start 112.3805 84.00732) (end 112.3805 70.62245) (width 0.2) (layer "F.Cu") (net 3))
 (segment (start 112.3805 70.62245) (end 122.6707 60.33225) (width 0.2) (layer "F.Cu") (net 3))
 (segment (start 133.8459 56.087) (end 158.576 56.087) (width 0.2) (layer "F.Cu") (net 3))
 (segment (start 172.4025 80.80375) (end 172.4025 83.793064) (width 0.2) (layer "F.Cu") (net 3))
 (segment (start 114.46893 86.09575) (end 112.3805 84.00732) (width 0.2) (layer "F.Cu") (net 3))
 (segment (start 172.4025 83.793064) (end 170.099814 86.09575) (width 0.2) (layer "F.Cu") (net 3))
 (segment (start 122.6707 60.33225) (end 129.60065 60.33225) (width 0.2) (layer "F.Cu") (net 3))
 (segment (start 129.60065 60.33225) (end 133.8459 56.087) (width 0.2) (layer "F.Cu") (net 3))
 (segment (start 158.576 56.087) (end 159.639 57.15) (width 0.2) (layer "F.Cu") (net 3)))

